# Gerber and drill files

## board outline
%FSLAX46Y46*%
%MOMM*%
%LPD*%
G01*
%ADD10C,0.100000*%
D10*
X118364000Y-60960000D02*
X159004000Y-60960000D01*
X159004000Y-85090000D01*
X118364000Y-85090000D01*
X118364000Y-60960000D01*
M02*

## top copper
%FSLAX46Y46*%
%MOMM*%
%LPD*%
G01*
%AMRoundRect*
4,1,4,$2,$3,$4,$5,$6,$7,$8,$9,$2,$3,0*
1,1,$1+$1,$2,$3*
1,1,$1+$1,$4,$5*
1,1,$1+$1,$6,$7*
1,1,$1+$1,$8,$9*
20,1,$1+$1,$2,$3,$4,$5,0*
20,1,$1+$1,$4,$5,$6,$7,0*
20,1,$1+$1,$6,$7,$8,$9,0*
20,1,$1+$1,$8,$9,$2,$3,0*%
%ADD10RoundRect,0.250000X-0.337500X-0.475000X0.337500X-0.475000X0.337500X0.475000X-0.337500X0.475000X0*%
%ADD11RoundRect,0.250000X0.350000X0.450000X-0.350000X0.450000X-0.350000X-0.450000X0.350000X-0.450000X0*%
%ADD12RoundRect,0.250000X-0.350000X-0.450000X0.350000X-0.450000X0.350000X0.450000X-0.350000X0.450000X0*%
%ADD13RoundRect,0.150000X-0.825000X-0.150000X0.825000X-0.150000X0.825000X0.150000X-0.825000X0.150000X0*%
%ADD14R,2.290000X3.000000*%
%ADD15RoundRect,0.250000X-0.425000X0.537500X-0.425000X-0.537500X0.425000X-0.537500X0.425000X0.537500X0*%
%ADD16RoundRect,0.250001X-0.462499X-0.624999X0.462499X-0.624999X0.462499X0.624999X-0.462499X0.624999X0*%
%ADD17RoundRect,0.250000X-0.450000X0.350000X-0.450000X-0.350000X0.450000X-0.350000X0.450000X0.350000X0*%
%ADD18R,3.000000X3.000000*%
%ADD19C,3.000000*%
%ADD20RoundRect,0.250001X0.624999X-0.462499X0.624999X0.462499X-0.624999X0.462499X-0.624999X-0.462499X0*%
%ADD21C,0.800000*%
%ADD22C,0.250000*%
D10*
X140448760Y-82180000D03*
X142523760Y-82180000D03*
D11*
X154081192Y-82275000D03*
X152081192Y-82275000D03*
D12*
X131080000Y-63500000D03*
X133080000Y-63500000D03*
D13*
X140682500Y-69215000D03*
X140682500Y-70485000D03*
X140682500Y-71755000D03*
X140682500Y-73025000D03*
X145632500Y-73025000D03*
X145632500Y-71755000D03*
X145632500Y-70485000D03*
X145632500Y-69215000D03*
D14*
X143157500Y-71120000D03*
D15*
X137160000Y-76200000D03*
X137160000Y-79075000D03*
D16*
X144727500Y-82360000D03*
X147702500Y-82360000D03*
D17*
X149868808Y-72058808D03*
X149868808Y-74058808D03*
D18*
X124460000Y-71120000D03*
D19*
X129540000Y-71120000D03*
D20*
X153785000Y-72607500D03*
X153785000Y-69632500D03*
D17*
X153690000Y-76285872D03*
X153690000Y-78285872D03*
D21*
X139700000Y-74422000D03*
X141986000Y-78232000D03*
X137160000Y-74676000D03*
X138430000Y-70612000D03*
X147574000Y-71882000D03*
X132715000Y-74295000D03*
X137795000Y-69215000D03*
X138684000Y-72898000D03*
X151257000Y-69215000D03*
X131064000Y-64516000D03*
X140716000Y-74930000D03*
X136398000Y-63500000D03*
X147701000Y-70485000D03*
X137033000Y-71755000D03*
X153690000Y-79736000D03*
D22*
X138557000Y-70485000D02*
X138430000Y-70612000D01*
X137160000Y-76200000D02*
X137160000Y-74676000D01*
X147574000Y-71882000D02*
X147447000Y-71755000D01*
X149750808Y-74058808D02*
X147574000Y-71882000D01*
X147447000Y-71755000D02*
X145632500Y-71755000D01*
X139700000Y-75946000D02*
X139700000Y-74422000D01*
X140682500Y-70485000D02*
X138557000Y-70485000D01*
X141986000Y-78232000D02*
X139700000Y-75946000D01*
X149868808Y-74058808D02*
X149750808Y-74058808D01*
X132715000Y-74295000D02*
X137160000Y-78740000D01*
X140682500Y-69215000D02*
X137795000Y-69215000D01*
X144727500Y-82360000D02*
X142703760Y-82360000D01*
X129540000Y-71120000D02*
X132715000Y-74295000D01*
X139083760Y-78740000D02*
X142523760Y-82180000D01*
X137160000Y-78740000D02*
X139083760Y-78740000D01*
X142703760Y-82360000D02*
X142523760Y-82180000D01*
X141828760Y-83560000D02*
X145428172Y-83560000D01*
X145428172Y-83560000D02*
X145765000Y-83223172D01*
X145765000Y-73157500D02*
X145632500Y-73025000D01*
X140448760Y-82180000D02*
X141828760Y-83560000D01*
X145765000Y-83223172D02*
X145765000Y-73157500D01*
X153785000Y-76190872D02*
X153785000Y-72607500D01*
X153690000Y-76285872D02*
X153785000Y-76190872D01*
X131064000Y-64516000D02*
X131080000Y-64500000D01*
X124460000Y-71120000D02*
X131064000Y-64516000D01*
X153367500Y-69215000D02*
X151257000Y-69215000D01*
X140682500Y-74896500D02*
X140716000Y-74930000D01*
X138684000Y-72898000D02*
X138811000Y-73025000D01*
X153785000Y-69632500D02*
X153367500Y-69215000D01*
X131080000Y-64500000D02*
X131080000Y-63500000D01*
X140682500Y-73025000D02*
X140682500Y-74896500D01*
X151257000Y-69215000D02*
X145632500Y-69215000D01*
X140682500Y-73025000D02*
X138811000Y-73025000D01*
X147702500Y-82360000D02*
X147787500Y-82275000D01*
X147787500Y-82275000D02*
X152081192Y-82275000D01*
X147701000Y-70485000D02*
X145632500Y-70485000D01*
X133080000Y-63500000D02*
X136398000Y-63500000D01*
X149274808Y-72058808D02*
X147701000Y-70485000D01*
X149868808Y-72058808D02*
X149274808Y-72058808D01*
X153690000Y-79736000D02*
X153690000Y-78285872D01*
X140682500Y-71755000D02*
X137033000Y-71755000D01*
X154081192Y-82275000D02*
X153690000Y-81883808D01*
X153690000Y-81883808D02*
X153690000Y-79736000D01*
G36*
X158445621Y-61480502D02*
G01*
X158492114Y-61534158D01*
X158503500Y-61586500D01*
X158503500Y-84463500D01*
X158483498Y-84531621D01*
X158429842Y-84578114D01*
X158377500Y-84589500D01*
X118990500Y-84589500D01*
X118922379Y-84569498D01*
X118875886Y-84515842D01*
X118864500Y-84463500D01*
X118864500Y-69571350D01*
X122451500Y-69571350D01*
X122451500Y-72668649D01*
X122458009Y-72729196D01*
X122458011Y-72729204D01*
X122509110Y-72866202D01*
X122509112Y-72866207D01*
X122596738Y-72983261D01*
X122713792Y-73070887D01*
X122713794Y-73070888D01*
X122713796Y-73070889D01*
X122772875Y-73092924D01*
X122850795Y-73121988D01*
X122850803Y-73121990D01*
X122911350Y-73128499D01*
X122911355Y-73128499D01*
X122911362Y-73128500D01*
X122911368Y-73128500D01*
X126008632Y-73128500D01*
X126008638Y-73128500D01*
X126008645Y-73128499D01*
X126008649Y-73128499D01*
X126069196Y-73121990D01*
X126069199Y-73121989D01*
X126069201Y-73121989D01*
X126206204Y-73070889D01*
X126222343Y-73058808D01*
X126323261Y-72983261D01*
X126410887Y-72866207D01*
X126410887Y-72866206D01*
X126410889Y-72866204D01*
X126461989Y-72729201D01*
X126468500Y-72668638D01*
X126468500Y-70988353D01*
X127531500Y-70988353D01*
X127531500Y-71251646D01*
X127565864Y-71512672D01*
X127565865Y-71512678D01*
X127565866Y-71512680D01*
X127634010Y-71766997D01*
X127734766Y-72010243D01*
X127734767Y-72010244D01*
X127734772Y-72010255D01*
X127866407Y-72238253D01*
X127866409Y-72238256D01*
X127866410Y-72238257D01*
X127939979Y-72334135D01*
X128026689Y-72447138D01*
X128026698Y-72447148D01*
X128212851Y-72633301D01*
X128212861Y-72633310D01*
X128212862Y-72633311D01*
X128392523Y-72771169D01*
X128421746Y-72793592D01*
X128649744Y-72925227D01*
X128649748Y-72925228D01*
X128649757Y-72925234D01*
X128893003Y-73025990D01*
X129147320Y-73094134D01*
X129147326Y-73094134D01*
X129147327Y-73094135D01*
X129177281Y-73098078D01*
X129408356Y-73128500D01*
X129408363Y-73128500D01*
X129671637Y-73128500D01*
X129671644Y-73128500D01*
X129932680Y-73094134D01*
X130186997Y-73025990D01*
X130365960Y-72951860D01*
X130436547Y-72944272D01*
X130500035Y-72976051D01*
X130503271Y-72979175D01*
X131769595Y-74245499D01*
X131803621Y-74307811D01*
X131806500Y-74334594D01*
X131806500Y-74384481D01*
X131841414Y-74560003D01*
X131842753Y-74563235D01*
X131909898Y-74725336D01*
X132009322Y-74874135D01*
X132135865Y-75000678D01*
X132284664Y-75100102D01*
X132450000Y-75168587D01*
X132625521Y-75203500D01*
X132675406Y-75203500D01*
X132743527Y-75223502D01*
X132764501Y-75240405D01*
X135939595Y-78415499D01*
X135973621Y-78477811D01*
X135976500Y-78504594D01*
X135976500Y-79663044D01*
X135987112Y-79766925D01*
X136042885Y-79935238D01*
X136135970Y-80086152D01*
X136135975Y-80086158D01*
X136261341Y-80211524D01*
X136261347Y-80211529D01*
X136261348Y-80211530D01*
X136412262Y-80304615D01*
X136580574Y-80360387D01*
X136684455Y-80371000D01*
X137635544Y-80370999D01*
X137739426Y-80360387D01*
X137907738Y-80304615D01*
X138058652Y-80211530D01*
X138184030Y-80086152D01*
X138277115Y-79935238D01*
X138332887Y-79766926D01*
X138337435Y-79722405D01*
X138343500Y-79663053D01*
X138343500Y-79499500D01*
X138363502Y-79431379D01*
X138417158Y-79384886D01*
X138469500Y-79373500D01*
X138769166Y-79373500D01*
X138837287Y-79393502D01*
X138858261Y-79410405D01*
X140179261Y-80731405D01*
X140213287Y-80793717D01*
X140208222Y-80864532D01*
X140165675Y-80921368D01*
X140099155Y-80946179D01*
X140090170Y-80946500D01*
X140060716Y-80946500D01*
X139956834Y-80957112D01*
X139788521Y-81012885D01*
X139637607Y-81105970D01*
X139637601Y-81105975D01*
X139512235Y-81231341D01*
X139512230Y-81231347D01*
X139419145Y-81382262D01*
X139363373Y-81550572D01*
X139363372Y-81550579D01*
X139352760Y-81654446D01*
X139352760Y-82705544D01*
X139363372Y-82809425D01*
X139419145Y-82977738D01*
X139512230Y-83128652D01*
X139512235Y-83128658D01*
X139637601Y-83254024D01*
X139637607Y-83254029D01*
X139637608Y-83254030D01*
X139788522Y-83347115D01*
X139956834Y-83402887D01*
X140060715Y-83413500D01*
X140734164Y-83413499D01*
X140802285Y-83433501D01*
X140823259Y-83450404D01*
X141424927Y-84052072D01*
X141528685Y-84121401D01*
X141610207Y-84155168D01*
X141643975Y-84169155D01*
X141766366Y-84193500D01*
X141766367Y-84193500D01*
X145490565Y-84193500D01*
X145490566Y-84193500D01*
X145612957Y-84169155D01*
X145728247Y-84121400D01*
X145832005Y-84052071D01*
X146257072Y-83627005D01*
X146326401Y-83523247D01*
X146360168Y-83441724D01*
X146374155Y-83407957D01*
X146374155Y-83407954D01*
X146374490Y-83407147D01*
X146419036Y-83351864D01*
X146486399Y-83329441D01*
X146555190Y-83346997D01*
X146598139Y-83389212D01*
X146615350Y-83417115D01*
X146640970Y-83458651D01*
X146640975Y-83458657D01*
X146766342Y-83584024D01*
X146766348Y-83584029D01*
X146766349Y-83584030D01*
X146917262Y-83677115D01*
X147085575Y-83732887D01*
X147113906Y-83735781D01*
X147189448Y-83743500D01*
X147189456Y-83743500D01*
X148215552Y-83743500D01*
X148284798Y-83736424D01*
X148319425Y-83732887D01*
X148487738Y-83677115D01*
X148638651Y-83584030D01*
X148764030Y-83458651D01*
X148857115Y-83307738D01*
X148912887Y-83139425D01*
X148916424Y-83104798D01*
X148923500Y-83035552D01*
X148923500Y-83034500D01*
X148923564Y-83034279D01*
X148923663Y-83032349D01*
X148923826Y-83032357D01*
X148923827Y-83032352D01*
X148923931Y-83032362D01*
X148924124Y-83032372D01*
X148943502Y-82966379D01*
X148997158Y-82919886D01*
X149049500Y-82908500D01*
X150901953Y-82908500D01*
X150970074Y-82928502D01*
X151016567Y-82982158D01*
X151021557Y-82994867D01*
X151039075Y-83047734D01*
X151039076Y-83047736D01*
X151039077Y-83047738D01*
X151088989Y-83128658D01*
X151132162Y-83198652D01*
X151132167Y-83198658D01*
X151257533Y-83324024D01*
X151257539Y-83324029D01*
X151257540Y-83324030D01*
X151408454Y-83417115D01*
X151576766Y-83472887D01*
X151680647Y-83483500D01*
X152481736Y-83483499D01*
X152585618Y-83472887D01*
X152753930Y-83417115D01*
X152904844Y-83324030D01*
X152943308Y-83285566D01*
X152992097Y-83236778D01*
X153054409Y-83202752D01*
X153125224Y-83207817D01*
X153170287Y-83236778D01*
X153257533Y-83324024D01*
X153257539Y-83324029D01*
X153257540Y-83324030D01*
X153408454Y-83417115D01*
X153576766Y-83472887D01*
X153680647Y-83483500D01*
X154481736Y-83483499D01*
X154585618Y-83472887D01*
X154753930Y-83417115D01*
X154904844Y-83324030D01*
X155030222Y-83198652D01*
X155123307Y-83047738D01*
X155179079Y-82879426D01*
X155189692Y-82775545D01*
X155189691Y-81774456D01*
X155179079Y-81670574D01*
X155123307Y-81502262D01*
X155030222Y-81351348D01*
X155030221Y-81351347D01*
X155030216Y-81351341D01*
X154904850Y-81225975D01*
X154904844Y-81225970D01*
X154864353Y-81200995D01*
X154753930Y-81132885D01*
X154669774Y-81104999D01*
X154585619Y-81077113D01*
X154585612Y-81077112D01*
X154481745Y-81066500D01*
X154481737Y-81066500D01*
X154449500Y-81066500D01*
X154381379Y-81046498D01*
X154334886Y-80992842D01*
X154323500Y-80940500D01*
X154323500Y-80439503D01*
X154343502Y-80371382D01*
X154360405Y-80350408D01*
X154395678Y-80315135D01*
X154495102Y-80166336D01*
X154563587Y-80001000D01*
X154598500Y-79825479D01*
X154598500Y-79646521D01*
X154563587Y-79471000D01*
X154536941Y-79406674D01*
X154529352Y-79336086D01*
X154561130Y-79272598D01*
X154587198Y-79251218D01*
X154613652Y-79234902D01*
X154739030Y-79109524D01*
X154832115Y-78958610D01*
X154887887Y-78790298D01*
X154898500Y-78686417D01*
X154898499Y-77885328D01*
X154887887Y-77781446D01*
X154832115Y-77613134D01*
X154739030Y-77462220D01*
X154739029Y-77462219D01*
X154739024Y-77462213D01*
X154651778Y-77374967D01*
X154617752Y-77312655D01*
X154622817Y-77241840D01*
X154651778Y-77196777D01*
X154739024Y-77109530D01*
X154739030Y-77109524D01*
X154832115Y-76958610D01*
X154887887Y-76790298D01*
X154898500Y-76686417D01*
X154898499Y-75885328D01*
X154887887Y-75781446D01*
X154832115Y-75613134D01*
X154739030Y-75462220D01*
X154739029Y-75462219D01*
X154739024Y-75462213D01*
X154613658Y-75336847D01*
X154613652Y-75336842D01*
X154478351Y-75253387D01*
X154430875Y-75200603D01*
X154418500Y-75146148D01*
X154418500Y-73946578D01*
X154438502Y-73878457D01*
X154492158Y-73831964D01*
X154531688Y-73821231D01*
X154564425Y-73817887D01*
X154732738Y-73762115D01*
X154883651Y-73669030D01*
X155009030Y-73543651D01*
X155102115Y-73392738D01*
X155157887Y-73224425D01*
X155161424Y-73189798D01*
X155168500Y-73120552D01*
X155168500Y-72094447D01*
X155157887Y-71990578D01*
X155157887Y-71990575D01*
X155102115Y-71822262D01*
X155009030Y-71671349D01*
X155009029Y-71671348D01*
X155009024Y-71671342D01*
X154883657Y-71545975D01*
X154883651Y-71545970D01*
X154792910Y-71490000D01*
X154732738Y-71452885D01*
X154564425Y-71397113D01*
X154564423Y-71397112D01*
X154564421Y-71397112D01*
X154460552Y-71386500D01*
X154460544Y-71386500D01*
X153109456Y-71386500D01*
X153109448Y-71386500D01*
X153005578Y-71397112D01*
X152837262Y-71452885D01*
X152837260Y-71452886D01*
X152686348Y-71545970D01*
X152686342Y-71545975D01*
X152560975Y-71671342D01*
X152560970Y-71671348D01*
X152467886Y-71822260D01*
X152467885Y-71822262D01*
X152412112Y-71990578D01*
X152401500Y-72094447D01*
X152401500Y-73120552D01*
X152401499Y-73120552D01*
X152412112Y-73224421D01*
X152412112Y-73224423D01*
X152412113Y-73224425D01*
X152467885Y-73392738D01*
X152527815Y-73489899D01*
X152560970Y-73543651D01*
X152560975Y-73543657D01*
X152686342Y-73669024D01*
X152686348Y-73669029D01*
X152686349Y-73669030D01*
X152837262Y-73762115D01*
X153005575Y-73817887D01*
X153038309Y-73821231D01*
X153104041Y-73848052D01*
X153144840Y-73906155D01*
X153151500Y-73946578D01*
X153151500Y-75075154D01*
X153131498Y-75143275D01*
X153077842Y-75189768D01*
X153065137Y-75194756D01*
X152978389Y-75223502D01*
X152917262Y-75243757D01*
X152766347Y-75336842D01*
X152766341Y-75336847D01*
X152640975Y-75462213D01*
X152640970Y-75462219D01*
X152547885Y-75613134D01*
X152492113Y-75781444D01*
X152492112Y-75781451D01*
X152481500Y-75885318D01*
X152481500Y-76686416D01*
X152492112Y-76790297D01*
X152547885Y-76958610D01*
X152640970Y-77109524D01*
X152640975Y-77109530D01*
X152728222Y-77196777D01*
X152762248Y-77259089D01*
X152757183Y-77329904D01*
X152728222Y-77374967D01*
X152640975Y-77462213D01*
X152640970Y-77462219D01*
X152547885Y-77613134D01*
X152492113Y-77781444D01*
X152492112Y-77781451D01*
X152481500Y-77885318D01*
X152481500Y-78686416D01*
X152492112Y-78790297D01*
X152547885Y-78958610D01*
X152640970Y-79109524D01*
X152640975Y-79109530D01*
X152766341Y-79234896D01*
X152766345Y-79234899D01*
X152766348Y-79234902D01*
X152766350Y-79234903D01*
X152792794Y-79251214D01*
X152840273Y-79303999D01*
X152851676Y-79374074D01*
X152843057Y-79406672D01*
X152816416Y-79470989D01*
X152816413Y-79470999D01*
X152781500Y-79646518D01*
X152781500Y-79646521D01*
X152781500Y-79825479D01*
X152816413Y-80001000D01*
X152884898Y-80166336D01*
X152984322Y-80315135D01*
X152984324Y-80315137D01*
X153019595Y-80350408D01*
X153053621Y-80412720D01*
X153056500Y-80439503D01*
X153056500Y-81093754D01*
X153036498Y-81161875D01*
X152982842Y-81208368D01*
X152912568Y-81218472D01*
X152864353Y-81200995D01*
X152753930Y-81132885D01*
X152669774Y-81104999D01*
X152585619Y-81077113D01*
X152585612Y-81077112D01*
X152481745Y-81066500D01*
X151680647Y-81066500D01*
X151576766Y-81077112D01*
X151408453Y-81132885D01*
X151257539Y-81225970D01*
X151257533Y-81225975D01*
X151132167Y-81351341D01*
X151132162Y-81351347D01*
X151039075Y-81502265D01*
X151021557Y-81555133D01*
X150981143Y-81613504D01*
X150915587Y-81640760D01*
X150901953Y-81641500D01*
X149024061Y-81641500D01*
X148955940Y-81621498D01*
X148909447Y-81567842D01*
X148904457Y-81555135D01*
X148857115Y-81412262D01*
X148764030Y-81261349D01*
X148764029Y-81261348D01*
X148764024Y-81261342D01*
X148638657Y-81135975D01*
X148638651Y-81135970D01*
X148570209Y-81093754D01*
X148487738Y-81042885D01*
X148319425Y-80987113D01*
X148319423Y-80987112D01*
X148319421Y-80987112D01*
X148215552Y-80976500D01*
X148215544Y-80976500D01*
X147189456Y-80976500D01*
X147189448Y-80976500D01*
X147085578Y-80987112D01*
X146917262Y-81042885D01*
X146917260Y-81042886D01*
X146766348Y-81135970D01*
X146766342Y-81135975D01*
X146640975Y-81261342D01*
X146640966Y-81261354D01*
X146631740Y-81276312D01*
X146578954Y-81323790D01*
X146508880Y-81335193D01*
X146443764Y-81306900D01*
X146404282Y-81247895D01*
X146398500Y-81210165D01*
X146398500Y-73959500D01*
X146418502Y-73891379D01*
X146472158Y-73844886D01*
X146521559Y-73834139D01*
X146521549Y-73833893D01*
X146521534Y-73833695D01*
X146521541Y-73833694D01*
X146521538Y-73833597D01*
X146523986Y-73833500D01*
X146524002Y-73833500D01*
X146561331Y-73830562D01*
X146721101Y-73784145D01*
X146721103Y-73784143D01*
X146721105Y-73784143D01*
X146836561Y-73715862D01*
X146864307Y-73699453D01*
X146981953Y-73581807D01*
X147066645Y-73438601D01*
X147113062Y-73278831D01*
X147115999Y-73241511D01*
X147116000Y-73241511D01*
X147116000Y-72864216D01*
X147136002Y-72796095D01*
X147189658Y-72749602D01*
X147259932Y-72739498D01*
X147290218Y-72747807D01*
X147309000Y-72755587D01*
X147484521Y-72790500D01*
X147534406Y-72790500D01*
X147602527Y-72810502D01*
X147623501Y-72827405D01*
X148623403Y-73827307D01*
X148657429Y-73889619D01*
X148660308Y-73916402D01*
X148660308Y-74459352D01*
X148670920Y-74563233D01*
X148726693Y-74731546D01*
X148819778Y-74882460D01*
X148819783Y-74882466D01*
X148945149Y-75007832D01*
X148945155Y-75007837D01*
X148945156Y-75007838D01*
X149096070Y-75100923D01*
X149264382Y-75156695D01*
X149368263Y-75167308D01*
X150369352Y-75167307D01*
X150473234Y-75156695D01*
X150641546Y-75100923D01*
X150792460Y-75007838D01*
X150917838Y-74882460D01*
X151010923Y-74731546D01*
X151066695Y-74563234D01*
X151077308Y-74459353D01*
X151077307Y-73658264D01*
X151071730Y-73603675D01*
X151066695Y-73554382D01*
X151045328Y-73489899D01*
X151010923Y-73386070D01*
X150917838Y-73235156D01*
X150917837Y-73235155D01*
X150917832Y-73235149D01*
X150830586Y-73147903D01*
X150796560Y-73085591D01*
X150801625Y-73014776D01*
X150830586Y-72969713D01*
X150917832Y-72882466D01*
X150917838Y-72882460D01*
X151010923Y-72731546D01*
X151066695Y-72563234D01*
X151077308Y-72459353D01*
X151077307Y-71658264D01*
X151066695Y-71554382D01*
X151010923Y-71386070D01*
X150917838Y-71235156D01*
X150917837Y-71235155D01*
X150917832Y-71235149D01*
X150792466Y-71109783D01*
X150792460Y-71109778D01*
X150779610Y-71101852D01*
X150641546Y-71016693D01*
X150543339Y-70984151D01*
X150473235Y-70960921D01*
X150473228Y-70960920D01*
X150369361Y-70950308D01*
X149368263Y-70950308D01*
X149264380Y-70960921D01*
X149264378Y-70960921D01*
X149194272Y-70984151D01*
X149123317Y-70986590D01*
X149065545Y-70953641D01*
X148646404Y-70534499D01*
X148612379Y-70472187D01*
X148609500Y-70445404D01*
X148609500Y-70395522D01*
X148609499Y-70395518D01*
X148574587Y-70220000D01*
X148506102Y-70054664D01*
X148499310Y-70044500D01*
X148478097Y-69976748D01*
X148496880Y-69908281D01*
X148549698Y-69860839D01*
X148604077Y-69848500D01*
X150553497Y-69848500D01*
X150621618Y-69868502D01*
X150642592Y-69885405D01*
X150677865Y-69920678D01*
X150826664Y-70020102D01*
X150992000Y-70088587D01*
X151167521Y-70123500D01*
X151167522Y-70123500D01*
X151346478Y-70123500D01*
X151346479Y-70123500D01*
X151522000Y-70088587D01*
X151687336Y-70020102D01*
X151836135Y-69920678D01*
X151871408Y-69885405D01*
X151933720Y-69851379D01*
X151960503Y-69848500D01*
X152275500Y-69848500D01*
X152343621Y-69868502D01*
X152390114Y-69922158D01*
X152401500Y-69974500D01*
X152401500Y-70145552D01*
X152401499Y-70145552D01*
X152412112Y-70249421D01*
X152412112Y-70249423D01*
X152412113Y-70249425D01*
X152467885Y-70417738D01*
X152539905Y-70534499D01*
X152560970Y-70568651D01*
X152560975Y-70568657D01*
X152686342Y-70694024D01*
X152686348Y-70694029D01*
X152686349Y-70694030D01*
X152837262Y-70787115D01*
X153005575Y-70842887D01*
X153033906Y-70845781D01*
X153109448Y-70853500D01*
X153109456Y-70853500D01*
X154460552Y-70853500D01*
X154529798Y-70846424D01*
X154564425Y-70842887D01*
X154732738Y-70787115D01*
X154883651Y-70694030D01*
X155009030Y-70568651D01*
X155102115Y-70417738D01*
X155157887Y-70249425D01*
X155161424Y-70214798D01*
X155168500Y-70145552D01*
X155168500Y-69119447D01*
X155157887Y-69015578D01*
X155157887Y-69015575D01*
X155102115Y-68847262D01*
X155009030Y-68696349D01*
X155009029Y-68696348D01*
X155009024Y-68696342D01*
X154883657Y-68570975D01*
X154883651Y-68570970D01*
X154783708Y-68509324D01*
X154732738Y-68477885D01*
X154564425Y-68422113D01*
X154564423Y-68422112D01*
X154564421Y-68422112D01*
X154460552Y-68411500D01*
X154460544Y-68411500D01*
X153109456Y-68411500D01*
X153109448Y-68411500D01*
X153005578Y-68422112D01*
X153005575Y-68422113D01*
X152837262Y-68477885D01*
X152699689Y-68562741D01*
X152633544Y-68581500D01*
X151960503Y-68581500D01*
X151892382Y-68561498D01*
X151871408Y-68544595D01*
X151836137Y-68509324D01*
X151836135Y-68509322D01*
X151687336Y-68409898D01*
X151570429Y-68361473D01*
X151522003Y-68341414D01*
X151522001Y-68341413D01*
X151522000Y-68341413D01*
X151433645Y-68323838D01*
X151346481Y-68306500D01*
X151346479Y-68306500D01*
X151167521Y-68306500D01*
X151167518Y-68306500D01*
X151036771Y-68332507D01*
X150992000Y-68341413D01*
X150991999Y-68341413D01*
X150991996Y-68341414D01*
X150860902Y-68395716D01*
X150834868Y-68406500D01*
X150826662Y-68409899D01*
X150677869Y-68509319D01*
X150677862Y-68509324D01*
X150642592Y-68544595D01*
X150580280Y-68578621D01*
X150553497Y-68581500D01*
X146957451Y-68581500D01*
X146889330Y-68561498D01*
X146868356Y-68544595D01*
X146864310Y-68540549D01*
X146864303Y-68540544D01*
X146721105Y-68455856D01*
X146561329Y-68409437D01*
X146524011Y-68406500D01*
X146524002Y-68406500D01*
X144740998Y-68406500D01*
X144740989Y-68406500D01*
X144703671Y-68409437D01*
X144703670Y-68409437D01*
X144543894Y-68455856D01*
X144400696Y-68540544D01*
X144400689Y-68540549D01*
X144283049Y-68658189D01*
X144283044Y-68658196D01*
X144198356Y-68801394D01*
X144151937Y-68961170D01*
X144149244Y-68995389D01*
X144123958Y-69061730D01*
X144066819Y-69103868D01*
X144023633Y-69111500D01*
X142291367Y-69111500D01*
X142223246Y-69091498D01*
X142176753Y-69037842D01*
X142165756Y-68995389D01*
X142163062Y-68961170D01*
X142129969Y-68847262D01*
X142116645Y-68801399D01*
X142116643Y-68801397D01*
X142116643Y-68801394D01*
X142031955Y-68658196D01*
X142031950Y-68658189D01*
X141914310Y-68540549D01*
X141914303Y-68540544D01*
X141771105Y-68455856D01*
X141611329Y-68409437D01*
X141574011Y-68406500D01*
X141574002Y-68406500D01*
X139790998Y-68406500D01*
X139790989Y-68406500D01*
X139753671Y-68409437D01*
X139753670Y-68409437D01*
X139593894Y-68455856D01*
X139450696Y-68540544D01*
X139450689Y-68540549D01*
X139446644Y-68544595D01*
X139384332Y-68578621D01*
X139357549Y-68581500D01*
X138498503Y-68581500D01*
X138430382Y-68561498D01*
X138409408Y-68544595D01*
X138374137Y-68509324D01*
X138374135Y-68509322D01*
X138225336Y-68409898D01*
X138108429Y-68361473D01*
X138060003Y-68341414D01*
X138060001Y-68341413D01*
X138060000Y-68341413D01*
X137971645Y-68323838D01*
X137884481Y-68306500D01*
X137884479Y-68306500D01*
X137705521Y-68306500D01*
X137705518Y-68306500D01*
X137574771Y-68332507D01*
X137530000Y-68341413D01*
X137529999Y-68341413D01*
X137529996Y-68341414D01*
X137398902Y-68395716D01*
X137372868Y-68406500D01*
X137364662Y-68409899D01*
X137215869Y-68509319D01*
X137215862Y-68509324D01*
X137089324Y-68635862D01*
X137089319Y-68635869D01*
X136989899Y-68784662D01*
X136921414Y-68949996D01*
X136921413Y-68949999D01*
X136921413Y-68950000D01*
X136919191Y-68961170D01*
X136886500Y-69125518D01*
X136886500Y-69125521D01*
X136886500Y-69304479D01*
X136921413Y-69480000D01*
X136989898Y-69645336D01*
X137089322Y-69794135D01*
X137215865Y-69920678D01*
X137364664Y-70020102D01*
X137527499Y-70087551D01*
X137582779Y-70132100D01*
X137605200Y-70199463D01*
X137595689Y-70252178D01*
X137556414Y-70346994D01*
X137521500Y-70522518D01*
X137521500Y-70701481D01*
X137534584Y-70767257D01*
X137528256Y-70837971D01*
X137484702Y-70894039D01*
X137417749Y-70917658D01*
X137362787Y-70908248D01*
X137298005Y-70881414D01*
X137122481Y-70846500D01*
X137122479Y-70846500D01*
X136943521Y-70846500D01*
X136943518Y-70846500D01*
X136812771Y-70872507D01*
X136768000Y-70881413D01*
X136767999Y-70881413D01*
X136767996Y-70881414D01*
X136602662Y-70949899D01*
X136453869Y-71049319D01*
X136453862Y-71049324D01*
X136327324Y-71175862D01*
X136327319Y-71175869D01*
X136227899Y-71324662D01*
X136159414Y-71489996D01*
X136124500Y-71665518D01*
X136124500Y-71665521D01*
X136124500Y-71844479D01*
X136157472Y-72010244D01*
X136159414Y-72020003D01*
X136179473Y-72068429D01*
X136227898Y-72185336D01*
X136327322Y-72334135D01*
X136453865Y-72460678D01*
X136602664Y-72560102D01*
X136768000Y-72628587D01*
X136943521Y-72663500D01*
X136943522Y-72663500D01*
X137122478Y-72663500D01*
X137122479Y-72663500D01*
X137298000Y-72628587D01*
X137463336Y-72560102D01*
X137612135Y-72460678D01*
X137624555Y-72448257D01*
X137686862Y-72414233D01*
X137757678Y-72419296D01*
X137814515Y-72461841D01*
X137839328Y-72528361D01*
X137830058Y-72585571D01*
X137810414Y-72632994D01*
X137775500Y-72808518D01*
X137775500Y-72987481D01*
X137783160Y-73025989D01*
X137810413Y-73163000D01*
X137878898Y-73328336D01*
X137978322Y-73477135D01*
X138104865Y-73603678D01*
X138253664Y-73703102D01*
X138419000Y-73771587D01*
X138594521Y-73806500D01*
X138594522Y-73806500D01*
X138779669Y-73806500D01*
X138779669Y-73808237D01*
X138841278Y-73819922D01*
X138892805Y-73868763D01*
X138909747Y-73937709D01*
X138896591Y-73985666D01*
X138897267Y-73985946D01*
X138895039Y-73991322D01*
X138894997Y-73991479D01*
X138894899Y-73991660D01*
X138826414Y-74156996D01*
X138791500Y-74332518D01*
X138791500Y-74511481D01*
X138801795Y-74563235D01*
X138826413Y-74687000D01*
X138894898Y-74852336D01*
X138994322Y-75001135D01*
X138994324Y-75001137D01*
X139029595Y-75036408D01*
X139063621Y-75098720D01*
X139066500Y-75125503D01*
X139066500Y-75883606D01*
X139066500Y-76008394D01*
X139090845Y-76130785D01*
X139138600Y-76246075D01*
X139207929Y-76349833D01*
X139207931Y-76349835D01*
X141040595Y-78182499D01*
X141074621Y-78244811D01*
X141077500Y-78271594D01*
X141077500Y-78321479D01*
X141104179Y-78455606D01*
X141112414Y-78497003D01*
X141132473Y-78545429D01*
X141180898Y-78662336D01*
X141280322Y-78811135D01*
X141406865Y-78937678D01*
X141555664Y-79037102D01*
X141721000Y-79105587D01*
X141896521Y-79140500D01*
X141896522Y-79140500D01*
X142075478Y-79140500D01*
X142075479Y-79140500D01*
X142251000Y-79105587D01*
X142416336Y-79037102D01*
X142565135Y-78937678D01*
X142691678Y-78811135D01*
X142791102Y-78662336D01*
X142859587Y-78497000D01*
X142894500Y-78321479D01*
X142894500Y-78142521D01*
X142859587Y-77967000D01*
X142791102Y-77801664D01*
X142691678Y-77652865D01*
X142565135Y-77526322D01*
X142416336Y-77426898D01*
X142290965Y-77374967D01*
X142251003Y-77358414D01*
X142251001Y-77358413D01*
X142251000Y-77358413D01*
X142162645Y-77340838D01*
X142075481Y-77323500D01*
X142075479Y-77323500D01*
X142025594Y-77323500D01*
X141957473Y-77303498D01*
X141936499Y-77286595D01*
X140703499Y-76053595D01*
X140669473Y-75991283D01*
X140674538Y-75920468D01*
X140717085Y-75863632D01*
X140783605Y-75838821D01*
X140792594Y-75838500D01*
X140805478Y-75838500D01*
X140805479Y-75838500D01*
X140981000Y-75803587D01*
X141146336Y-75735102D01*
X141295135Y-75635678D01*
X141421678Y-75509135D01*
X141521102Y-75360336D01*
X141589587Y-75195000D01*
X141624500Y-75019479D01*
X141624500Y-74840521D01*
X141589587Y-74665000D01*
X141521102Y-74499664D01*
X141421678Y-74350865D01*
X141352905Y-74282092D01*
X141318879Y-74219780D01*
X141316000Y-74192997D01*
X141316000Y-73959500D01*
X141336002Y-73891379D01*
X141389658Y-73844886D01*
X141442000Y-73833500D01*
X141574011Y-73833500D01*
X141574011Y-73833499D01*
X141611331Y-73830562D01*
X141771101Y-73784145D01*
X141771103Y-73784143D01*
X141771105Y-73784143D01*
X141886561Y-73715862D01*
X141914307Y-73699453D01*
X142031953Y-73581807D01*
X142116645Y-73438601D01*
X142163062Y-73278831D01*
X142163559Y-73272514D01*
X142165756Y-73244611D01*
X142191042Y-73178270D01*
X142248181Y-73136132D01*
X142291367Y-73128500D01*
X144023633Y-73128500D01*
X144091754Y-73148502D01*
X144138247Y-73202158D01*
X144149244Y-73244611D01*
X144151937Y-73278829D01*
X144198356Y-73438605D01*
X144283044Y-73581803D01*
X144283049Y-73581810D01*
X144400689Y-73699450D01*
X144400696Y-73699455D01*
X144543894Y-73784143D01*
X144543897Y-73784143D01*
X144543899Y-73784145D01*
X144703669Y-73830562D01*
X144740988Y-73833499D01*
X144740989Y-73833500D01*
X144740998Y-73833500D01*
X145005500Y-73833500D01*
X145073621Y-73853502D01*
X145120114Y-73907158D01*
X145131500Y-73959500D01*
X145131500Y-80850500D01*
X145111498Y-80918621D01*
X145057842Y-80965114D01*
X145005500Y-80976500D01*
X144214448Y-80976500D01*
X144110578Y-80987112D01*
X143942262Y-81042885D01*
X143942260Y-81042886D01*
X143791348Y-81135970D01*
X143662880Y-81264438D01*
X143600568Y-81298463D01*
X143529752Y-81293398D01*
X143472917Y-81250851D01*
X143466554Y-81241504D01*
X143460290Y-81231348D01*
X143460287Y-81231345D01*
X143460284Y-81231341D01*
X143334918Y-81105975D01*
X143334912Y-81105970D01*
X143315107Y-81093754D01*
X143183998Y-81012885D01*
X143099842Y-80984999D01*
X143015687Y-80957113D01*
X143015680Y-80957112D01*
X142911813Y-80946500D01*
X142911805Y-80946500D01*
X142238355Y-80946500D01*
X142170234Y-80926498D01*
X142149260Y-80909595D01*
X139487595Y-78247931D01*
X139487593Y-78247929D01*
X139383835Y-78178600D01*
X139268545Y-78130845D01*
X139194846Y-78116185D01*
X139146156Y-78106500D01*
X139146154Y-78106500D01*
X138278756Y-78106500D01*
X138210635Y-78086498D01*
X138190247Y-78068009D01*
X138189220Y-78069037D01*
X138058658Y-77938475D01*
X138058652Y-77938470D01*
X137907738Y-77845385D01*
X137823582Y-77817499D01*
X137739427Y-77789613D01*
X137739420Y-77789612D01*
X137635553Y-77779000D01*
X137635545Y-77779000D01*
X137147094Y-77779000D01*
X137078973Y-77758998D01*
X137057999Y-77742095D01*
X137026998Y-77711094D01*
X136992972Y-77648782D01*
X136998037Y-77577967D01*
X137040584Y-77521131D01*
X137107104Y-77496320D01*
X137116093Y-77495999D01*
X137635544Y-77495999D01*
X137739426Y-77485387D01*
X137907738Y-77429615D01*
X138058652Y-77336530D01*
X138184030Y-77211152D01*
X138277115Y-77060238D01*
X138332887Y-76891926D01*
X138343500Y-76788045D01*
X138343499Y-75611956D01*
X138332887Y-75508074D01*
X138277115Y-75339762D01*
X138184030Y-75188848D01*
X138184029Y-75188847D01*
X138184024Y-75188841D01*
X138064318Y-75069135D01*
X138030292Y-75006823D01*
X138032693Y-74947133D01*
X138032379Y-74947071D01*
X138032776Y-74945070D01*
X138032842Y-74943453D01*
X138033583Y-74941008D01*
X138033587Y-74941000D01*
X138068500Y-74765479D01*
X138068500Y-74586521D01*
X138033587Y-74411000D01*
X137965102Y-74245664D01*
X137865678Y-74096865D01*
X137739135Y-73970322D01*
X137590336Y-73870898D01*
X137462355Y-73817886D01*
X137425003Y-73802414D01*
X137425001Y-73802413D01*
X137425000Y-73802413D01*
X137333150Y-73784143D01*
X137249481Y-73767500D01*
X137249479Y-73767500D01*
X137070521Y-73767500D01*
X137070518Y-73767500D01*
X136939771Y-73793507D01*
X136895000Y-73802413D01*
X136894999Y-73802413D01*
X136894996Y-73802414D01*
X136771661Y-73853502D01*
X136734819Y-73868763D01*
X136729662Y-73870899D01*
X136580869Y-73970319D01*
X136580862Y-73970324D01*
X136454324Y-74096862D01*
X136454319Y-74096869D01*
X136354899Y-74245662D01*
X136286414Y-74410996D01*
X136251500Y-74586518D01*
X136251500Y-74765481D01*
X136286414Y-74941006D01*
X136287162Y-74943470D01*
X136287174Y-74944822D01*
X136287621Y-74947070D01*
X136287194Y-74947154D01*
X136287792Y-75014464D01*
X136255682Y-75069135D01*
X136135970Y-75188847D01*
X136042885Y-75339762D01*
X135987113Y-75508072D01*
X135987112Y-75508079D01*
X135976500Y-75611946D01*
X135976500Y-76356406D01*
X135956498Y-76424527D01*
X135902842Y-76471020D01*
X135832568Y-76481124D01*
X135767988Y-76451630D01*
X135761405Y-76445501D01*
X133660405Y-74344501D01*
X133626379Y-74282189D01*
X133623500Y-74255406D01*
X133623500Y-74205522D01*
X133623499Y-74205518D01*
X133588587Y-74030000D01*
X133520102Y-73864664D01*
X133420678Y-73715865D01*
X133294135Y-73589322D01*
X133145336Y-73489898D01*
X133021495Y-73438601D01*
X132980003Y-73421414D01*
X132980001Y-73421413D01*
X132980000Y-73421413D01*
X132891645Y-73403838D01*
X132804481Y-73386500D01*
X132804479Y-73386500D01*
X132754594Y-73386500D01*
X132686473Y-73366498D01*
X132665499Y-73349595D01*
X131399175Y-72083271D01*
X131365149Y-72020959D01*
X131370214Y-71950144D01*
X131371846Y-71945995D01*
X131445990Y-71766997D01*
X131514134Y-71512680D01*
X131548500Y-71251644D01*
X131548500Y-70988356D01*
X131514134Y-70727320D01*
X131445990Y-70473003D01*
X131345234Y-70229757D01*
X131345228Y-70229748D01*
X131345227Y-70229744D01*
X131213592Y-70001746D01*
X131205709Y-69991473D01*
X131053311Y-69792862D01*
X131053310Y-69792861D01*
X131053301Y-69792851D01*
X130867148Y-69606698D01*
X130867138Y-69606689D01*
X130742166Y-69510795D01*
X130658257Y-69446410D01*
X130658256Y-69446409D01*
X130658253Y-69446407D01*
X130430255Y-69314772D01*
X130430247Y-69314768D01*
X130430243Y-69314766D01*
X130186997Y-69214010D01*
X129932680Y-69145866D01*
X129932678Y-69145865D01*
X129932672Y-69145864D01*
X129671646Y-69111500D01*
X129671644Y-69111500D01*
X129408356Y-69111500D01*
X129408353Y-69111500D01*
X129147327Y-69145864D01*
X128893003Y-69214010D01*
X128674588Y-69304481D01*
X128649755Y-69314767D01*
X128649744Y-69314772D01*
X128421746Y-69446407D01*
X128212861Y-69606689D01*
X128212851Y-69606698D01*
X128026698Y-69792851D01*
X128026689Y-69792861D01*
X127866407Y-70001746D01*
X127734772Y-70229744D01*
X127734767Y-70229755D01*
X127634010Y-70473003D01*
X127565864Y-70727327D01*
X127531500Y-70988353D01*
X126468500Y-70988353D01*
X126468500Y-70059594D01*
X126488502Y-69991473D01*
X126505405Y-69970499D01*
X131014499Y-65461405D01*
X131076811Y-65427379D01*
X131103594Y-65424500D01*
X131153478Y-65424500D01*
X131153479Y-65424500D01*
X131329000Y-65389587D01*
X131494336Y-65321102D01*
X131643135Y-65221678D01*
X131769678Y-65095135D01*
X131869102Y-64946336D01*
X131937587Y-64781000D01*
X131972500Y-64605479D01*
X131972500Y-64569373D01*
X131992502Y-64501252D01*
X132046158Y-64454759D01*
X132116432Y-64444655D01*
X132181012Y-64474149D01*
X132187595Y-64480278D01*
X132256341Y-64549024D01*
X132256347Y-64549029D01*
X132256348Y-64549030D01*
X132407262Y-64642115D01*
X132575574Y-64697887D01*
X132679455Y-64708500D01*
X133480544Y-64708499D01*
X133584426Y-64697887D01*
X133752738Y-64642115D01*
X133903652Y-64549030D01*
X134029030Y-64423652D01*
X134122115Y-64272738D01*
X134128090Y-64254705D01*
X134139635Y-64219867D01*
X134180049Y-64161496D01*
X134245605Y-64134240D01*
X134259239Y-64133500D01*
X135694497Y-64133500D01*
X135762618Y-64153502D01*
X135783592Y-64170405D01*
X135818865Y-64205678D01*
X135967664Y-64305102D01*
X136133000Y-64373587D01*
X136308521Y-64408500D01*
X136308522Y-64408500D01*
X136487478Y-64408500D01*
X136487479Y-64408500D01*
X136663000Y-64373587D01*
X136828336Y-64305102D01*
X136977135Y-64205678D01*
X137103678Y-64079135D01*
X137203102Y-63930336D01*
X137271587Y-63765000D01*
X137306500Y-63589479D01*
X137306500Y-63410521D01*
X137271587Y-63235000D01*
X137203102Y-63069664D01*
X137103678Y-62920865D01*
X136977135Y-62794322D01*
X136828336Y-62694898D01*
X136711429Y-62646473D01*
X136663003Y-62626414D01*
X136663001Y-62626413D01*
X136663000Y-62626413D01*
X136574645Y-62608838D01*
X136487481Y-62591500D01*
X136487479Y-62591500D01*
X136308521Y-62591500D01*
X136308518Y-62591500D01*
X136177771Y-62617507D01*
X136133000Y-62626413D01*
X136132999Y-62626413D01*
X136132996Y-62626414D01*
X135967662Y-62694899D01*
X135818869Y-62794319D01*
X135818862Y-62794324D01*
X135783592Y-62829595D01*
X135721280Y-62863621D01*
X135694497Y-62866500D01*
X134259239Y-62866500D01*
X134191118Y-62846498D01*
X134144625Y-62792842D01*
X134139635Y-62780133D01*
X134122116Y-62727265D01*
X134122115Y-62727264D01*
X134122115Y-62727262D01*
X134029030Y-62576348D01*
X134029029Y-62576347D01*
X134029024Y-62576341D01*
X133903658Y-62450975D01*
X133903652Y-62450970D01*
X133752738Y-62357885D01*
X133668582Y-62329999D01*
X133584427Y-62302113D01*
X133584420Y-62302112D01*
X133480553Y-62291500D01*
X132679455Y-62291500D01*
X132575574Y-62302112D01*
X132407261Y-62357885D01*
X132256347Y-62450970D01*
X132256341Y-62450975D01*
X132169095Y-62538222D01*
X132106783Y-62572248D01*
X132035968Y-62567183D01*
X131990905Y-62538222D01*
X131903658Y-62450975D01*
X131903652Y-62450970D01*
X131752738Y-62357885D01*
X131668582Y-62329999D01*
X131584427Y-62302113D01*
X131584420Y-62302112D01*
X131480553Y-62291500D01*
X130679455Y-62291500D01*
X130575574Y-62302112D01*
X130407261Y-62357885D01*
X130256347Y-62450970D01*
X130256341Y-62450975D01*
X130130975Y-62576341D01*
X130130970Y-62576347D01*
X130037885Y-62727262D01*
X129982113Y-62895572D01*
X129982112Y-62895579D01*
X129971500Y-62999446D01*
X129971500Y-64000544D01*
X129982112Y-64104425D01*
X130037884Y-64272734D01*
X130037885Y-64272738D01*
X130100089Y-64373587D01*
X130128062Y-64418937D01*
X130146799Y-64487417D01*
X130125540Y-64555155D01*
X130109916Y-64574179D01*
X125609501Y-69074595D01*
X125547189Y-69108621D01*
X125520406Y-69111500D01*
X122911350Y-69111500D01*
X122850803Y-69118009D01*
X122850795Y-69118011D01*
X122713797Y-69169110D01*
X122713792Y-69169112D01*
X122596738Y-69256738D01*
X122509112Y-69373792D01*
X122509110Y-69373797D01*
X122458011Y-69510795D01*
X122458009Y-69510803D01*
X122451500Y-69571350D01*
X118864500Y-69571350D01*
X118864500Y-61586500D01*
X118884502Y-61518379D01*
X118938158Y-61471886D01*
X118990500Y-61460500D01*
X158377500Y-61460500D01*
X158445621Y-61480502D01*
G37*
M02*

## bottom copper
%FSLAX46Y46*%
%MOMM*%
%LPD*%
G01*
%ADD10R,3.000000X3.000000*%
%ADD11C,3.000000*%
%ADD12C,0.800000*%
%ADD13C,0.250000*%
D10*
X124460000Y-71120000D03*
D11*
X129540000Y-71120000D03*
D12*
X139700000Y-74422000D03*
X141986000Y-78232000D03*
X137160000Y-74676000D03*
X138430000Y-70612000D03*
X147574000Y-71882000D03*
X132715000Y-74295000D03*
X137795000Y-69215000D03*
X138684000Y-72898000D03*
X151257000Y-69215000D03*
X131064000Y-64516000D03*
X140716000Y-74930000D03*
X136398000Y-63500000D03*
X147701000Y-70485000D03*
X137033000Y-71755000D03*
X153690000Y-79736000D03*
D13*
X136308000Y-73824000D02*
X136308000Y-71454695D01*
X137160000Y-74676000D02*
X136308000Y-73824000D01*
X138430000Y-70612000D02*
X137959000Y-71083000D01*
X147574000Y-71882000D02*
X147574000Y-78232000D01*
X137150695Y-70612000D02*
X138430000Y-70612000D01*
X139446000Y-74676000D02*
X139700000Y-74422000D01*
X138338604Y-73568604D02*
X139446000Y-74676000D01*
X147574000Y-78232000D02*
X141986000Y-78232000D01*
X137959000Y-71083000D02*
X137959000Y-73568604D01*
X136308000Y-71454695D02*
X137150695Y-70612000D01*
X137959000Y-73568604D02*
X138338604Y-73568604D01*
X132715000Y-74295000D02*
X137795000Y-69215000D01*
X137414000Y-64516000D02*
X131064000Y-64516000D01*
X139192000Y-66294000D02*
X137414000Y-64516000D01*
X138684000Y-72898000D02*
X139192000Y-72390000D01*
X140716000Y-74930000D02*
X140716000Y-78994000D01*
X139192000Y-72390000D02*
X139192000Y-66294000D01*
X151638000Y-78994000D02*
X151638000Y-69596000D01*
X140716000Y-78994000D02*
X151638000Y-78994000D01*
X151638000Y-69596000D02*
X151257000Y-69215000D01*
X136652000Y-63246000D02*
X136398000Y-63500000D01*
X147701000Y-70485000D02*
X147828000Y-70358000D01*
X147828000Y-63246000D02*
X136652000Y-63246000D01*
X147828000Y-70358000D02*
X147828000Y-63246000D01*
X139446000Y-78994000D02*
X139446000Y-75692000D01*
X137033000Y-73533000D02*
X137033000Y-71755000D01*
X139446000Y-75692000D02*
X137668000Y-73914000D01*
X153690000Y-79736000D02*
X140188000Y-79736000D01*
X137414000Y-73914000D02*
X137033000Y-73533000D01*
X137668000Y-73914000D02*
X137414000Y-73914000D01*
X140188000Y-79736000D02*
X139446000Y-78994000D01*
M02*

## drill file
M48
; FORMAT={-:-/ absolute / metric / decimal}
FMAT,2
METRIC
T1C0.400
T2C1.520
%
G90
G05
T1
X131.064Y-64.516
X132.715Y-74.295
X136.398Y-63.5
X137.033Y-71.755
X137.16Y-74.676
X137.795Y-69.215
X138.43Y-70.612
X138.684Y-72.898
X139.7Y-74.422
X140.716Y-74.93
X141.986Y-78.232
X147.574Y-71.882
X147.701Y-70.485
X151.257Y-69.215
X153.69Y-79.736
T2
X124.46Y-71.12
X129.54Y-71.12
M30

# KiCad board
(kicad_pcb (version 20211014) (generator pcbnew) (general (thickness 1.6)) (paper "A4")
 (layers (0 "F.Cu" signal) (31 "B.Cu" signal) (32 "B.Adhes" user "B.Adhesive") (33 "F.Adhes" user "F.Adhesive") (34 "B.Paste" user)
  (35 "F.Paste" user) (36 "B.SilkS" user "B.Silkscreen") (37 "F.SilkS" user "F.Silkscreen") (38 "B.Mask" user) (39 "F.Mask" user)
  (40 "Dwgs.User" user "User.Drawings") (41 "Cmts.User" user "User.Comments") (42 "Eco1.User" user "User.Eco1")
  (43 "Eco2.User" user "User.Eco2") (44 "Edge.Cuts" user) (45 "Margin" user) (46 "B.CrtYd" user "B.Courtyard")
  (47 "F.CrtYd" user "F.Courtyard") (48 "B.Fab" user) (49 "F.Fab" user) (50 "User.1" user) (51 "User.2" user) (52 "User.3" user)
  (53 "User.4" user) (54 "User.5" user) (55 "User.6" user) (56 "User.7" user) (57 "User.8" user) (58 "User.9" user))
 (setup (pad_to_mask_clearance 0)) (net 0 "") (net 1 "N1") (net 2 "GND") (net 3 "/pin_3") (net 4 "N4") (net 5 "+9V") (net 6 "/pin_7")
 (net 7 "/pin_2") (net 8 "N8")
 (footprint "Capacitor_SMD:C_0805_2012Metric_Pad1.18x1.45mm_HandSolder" (layer "F.Cu") (at 141.48626 82.18)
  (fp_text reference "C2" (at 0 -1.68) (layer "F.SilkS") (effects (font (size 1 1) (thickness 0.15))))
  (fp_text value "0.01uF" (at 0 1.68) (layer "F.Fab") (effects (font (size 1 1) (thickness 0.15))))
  (pad "1" smd roundrect (at -1.0375 0) (size 1.175 1.45) (layers "F.Cu" "F.Paste" "F.Mask") (roundrect_rratio 0.2127659574) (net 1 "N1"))
  (pad "2" smd roundrect (at 1.0375 0) (size 1.175 1.45) (layers "F.Cu" "F.Paste" "F.Mask") (roundrect_rratio 0.2127659574) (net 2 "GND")))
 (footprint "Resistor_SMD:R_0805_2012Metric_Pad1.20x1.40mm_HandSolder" (layer "F.Cu") (at 153.081192 82.275 180)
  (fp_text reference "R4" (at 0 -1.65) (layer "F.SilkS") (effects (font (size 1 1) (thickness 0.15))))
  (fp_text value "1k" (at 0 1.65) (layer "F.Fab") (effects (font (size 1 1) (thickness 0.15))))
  (pad "1" smd roundrect (at -1 0 180) (size 1.2 1.4) (layers "F.Cu" "F.Paste" "F.Mask") (roundrect_rratio 0.2083333333) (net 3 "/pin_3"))
  (pad "2" smd roundrect (at 1 0 180) (size 1.2 1.4) (layers "F.Cu" "F.Paste" "F.Mask") (roundrect_rratio 0.2083333333) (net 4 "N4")))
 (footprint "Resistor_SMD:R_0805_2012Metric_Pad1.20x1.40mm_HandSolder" (layer "F.Cu") (at 132.08 63.5)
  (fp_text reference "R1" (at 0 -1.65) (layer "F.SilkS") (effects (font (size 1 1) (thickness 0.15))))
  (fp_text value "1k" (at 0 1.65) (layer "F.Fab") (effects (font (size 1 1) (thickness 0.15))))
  (pad "1" smd roundrect (at -1 0) (size 1.2 1.4) (layers "F.Cu" "F.Paste" "F.Mask") (roundrect_rratio 0.2083333333) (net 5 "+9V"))
  (pad "2" smd roundrect (at 1 0) (size 1.2 1.4) (layers "F.Cu" "F.Paste" "F.Mask") (roundrect_rratio 0.2083333333) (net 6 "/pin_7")))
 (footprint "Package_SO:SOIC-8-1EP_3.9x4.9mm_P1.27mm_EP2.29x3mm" (layer "F.Cu") (at 143.1575 71.12)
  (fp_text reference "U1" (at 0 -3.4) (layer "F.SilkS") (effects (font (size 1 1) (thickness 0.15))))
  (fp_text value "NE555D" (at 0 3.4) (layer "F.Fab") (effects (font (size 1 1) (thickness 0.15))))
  (pad "" smd roundrect (at 0.57 0.75) (size 0.92 1.21) (layers "F.Paste") (roundrect_rratio 0.25))
  (pad "" smd roundrect (at 0.57 -0.75) (size 0.92 1.21) (layers "F.Paste") (roundrect_rratio 0.25))
  (pad "" smd roundrect (at -0.57 -0.75) (size 0.92 1.21) (layers "F.Paste") (roundrect_rratio 0.25))
  (pad "" smd roundrect (at -0.57 0.75) (size 0.92 1.21) (layers "F.Paste") (roundrect_rratio 0.25))
  (pad "1" smd roundrect (at -2.475 -1.905) (size 1.95 0.6) (layers "F.Cu" "F.Paste" "F.Mask") (roundrect_rratio 0.25) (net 2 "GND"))
  (pad "2" smd roundrect (at -2.475 -0.635) (size 1.95 0.6) (layers "F.Cu" "F.Paste" "F.Mask") (roundrect_rratio 0.25) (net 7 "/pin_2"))
  (pad "3" smd roundrect (at -2.475 0.635) (size 1.95 0.6) (layers "F.Cu" "F.Paste" "F.Mask") (roundrect_rratio 0.25) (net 3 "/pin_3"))
  (pad "4" smd roundrect (at -2.475 1.905) (size 1.95 0.6) (layers "F.Cu" "F.Paste" "F.Mask") (roundrect_rratio 0.25) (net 5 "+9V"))
  (pad "5" smd roundrect (at 2.475 1.905) (size 1.95 0.6) (layers "F.Cu" "F.Paste" "F.Mask") (roundrect_rratio 0.25) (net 1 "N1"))
  (pad "6" smd roundrect (at 2.475 0.635) (size 1.95 0.6) (layers "F.Cu" "F.Paste" "F.Mask") (roundrect_rratio 0.25) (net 7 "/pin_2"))
  (pad "7" smd roundrect (at 2.475 -0.635) (size 1.95 0.6) (layers "F.Cu" "F.Paste" "F.Mask") (roundrect_rratio 0.25) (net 6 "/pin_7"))
  (pad "8" smd roundrect (at 2.475 -1.905) (size 1.95 0.6) (layers "F.Cu" "F.Paste" "F.Mask") (roundrect_rratio 0.25) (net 5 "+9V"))
  (pad "9" smd rect (at 0 0) (size 2.29 3) (layers "F.Cu" "F.Mask")))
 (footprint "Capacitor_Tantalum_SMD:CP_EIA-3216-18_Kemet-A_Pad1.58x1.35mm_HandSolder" (layer "F.Cu") (at 137.16 77.6375 -90)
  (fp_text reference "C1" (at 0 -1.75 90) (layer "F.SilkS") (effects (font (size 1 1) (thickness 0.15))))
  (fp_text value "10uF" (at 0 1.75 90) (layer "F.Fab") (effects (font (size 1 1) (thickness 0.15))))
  (pad "1" smd roundrect (at -1.4375 0 270) (size 1.575 1.35) (layers "F.Cu" "F.Paste" "F.Mask") (roundrect_rratio 0.1851851852)
   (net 7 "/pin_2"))
  (pad "2" smd roundrect (at 1.4375 0 270) (size 1.575 1.35) (layers "F.Cu" "F.Paste" "F.Mask") (roundrect_rratio 0.1851851852)
   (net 2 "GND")))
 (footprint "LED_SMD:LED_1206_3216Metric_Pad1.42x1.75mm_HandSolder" (layer "F.Cu") (at 146.215 82.36)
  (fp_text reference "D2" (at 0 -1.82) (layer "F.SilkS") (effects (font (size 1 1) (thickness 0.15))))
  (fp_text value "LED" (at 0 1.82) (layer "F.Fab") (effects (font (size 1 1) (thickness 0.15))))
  (pad "1" smd roundrect (at -1.4875 0) (size 1.425 1.75) (layers "F.Cu" "F.Paste" "F.Mask") (roundrect_rratio 0.1754392982) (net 2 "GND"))
  (pad "2" smd roundrect (at 1.4875 0) (size 1.425 1.75) (layers "F.Cu" "F.Paste" "F.Mask") (roundrect_rratio 0.1754392982) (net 4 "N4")))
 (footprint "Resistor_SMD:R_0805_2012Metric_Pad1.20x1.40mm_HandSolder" (layer "F.Cu") (at 149.868808 73.058808 -90)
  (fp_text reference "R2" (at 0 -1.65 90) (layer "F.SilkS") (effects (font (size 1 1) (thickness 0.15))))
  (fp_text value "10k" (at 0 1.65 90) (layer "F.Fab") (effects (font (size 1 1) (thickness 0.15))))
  (pad "1" smd roundrect (at -1 0 270) (size 1.2 1.4) (layers "F.Cu" "F.Paste" "F.Mask") (roundrect_rratio 0.2083333333) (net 6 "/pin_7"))
  (pad "2" smd roundrect (at 1 0 270) (size 1.2 1.4) (layers "F.Cu" "F.Paste" "F.Mask") (roundrect_rratio 0.2083333333) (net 7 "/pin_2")))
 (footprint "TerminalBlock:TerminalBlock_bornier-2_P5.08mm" (layer "F.Cu") (at 124.46 71.12)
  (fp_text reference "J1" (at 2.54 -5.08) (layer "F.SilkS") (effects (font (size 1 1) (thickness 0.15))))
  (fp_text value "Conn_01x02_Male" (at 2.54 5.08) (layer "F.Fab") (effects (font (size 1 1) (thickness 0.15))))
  (pad "1" thru_hole rect (at 0 0) (size 3 3) (drill 1.52) (layers *.Cu *.Mask) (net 5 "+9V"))
  (pad "2" thru_hole circle (at 5.08 0) (size 3 3) (drill 1.52) (layers *.Cu *.Mask) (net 2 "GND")))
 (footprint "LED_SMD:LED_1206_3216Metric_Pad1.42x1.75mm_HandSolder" (layer "F.Cu") (at 153.785 71.12 90)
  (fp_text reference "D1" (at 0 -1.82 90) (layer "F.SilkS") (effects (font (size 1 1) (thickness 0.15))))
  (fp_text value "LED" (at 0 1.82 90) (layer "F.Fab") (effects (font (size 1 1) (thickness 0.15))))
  (pad "1" smd roundrect (at -1.4875 0 90) (size 1.425 1.75) (layers "F.Cu" "F.Paste" "F.Mask") (roundrect_rratio 0.1754392982) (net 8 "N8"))
  (pad "2" smd roundrect (at 1.4875 0 90) (size 1.425 1.75) (layers "F.Cu" "F.Paste" "F.Mask") (roundrect_rratio 0.1754392982) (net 5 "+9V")))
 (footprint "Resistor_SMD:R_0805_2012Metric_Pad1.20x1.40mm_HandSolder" (layer "F.Cu") (at 153.69 77.285872 -90)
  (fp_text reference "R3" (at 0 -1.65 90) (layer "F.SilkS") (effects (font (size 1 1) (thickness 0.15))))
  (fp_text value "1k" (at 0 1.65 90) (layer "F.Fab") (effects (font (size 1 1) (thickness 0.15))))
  (pad "1" smd roundrect (at -1 0 270) (size 1.2 1.4) (layers "F.Cu" "F.Paste" "F.Mask") (roundrect_rratio 0.2083333333) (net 8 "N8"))
  (pad "2" smd roundrect (at 1 0 270) (size 1.2 1.4) (layers "F.Cu" "F.Paste" "F.Mask") (roundrect_rratio 0.2083333333) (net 3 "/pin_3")))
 (gr_rect (start 118.364 60.96) (end 159.004 85.09) (layer "Edge.Cuts") (width 0.1) (fill none))
 (segment (start 138.557 70.485) (end 138.43 70.612) (width 0.25) (layer "F.Cu") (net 7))
 (segment (start 137.16 76.2) (end 137.16 74.676) (width 0.25) (layer "F.Cu") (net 7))
 (segment (start 147.574 71.882) (end 147.447 71.755) (width 0.25) (layer "F.Cu") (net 7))
 (segment (start 149.750808 74.058808) (end 147.574 71.882) (width 0.25) (layer "F.Cu") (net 7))
 (segment (start 147.447 71.755) (end 145.6325 71.755) (width 0.25) (layer "F.Cu") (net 7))
 (segment (start 139.7 75.946) (end 139.7 74.422) (width 0.25) (layer "F.Cu") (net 7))
 (segment (start 140.6825 70.485) (end 138.557 70.485) (width 0.25) (layer "F.Cu") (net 7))
 (segment (start 141.986 78.232) (end 139.7 75.946) (width 0.25) (layer "F.Cu") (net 7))
 (segment (start 149.868808 74.058808) (end 149.750808 74.058808) (width 0.25) (layer "F.Cu") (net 7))
 (via (at 139.7 74.422) (size 0.8) (drill 0.4) (layers "F.Cu" "B.Cu") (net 7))
 (via (at 141.986 78.232) (size 0.8) (drill 0.4) (layers "F.Cu" "B.Cu") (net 7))
 (via (at 137.16 74.676) (size 0.8) (drill 0.4) (layers "F.Cu" "B.Cu") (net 7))
 (via (at 138.43 70.612) (size 0.8) (drill 0.4) (layers "F.Cu" "B.Cu") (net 7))
 (via (at 147.574 71.882) (size 0.8) (drill 0.4) (layers "F.Cu" "B.Cu") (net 7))
 (segment (start 136.308 73.824) (end 136.308 71.454695) (width 0.25) (layer "B.Cu") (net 7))
 (segment (start 137.16 74.676) (end 136.308 73.824) (width 0.25) (layer "B.Cu") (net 7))
 (segment (start 138.43 70.612) (end 137.959 71.083) (width 0.25) (layer "B.Cu") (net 7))
 (segment (start 147.574 71.882) (end 147.574 78.232) (width 0.25) (layer "B.Cu") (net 7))
 (segment (start 137.150695 70.612) (end 138.43 70.612) (width 0.25) (layer "B.Cu") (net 7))
 (segment (start 139.446 74.676) (end 139.7 74.422) (width 0.25) (layer "B.Cu") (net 7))
 (segment (start 138.338604 73.568604) (end 139.446 74.676) (width 0.25) (layer "B.Cu") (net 7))
 (segment (start 147.574 78.232) (end 141.986 78.232) (width 0.25) (layer "B.Cu") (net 7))
 (segment (start 137.959 71.083) (end 137.959 73.568604) (width 0.25) (layer "B.Cu") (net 7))
 (segment (start 136.308 71.454695) (end 137.150695 70.612) (width 0.25) (layer "B.Cu") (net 7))
 (segment (start 137.959 73.568604) (end 138.338604 73.568604) (width 0.25) (layer "B.Cu") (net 7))
 (segment (start 132.715 74.295) (end 137.16 78.74) (width 0.25) (layer "F.Cu") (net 2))
 (segment (start 140.6825 69.215) (end 137.795 69.215) (width 0.25) (layer "F.Cu") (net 2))
 (segment (start 144.7275 82.36) (end 142.70376 82.36) (width 0.25) (layer "F.Cu") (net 2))
 (segment (start 129.54 71.12) (end 132.715 74.295) (width 0.25) (layer "F.Cu") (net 2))
 (segment (start 139.08376 78.74) (end 142.52376 82.18) (width 0.25) (layer "F.Cu") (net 2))
 (segment (start 137.16 78.74) (end 139.08376 78.74) (width 0.25) (layer "F.Cu") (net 2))
 (segment (start 142.70376 82.36) (end 142.52376 82.18) (width 0.25) (layer "F.Cu") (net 2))
 (via (at 132.715 74.295) (size 0.8) (drill 0.4) (layers "F.Cu" "B.Cu") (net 2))
 (via (at 137.795 69.215) (size 0.8) (drill 0.4) (layers "F.Cu" "B.Cu") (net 2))
 (segment (start 132.715 74.295) (end 137.795 69.215) (width 0.25) (layer "B.Cu") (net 2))
 (segment (start 141.82876 83.56) (end 145.428172 83.56) (width 0.25) (layer "F.Cu") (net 1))
 (segment (start 145.428172 83.56) (end 145.765 83.223172) (width 0.25) (layer "F.Cu") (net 1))
 (segment (start 145.765 73.1575) (end 145.6325 73.025) (width 0.25) (layer "F.Cu") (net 1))
 (segment (start 140.44876 82.18) (end 141.82876 83.56) (width 0.25) (layer "F.Cu") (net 1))
 (segment (start 145.765 83.223172) (end 145.765 73.1575) (width 0.25) (layer "F.Cu") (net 1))
 (segment (start 153.785 76.190872) (end 153.785 72.6075) (width 0.25) (layer "F.Cu") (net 8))
 (segment (start 153.69 76.285872) (end 153.785 76.190872) (width 0.25) (layer "F.Cu") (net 8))
 (segment (start 131.064 64.516) (end 131.08 64.5) (width 0.25) (layer "F.Cu") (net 5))
 (segment (start 124.46 71.12) (end 131.064 64.516) (width 0.25) (layer "F.Cu") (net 5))
 (segment (start 153.3675 69.215) (end 151.257 69.215) (width 0.25) (layer "F.Cu") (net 5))
 (segment (start 140.6825 74.8965) (end 140.716 74.93) (width 0.25) (layer "F.Cu") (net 5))
 (segment (start 138.684 72.898) (end 138.811 73.025) (width 0.25) (layer "F.Cu") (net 5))
 (segment (start 153.785 69.6325) (end 153.3675 69.215) (width 0.25) (layer "F.Cu") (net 5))
 (segment (start 131.08 64.5) (end 131.08 63.5) (width 0.25) (layer "F.Cu") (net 5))
 (segment (start 140.6825 73.025) (end 140.6825 74.8965) (width 0.25) (layer "F.Cu") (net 5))
 (segment (start 151.257 69.215) (end 145.6325 69.215) (width 0.25) (layer "F.Cu") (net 5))
 (segment (start 140.6825 73.025) (end 138.811 73.025) (width 0.25) (layer "F.Cu") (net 5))
 (via (at 138.684 72.898) (size 0.8) (drill 0.4) (layers "F.Cu" "B.Cu") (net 5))
 (via (at 151.257 69.215) (size 0.8) (drill 0.4) (layers "F.Cu" "B.Cu") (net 5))
 (via (at 131.064 64.516) (size 0.8) (drill 0.4) (layers "F.Cu" "B.Cu") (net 5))
 (via (at 140.716 74.93) (size 0.8) (drill 0.4) (layers "F.Cu" "B.Cu") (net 5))
 (segment (start 137.414 64.516) (end 131.064 64.516) (width 0.25) (layer "B.Cu") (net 5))
 (segment (start 139.192 66.294) (end 137.414 64.516) (width 0.25) (layer "B.Cu") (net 5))
 (segment (start 138.684 72.898) (end 139.192 72.39) (width 0.25) (layer "B.Cu") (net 5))
 (segment (start 140.716 74.93) (end 140.716 78.994) (width 0.25) (layer "B.Cu") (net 5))
 (segment (start 139.192 72.39) (end 139.192 66.294) (width 0.25) (layer "B.Cu") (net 5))
 (segment (start 151.638 78.994) (end 151.638 69.596) (width 0.25) (layer "B.Cu") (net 5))
 (segment (start 140.716 78.994) (end 151.638 78.994) (width 0.25) (layer "B.Cu") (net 5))
 (segment (start 151.638 69.596) (end 151.257 69.215) (width 0.25) (layer "B.Cu") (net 5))
 (segment (start 147.7025 82.36) (end 147.7875 82.275) (width 0.25) (layer "F.Cu") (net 4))
 (segment (start 147.7875 82.275) (end 152.081192 82.275) (width 0.25) (layer "F.Cu") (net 4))
 (segment (start 147.701 70.485) (end 145.6325 70.485) (width 0.25) (layer "F.Cu") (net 6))
 (segment (start 133.08 63.5) (end 136.398 63.5) (width 0.25) (layer "F.Cu") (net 6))
 (segment (start 149.274808 72.058808) (end 147.701 70.485) (width 0.25) (layer "F.Cu") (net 6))
 (segment (start 149.868808 72.058808) (end 149.274808 72.058808) (width 0.25) (layer "F.Cu") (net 6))
 (via (at 136.398 63.5) (size 0.8) (drill 0.4) (layers "F.Cu" "B.Cu") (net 6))
 (via (at 147.701 70.485) (size 0.8) (drill 0.4) (layers "F.Cu" "B.Cu") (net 6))
 (segment (start 136.652 63.246) (end 136.398 63.5) (width 0.25) (layer "B.Cu") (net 6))
 (segment (start 147.701 70.485) (end 147.828 70.358) (width 0.25) (layer "B.Cu") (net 6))
 (segment (start 147.828 63.246) (end 136.652 63.246) (width 0.25) (layer "B.Cu") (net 6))
 (segment (start 147.828 70.358) (end 147.828 63.246) (width 0.25) (layer "B.Cu") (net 6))
 (segment (start 153.69 79.736) (end 153.69 78.285872) (width 0.25) (layer "F.Cu") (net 3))
 (segment (start 140.6825 71.755) (end 137.033 71.755) (width 0.25) (layer "F.Cu") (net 3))
 (segment (start 154.081192 82.275) (end 153.69 81.883808) (width 0.25) (layer "F.Cu") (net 3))
 (segment (start 153.69 81.883808) (end 153.69 79.736) (width 0.25) (layer "F.Cu") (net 3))
 (via (at 137.033 71.755) (size 0.8) (drill 0.4) (layers "F.Cu" "B.Cu") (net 3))
 (via (at 153.69 79.736) (size 0.8) (drill 0.4) (layers "F.Cu" "B.Cu") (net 3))
 (segment (start 139.446 78.994) (end 139.446 75.692) (width 0.25) (layer "B.Cu") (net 3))
 (segment (start 137.033 73.533) (end 137.033 71.755) (width 0.25) (layer "B.Cu") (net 3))
 (segment (start 139.446 75.692) (end 137.668 73.914) (width 0.25) (layer "B.Cu") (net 3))
 (segment (start 153.69 79.736) (end 140.188 79.736) (width 0.25) (layer "B.Cu") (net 3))
 (segment (start 137.414 73.914) (end 137.033 73.533) (width 0.25) (layer "B.Cu") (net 3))
 (segment (start 137.668 73.914) (end 137.414 73.914) (width 0.25) (layer "B.Cu") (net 3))
 (segment (start 140.188 79.736) (end 139.446 78.994) (width 0.25) (layer "B.Cu") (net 3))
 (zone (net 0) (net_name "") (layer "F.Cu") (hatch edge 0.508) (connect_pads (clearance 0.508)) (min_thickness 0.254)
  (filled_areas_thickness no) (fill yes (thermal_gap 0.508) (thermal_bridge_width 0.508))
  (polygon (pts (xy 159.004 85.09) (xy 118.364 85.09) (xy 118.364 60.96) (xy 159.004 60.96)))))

